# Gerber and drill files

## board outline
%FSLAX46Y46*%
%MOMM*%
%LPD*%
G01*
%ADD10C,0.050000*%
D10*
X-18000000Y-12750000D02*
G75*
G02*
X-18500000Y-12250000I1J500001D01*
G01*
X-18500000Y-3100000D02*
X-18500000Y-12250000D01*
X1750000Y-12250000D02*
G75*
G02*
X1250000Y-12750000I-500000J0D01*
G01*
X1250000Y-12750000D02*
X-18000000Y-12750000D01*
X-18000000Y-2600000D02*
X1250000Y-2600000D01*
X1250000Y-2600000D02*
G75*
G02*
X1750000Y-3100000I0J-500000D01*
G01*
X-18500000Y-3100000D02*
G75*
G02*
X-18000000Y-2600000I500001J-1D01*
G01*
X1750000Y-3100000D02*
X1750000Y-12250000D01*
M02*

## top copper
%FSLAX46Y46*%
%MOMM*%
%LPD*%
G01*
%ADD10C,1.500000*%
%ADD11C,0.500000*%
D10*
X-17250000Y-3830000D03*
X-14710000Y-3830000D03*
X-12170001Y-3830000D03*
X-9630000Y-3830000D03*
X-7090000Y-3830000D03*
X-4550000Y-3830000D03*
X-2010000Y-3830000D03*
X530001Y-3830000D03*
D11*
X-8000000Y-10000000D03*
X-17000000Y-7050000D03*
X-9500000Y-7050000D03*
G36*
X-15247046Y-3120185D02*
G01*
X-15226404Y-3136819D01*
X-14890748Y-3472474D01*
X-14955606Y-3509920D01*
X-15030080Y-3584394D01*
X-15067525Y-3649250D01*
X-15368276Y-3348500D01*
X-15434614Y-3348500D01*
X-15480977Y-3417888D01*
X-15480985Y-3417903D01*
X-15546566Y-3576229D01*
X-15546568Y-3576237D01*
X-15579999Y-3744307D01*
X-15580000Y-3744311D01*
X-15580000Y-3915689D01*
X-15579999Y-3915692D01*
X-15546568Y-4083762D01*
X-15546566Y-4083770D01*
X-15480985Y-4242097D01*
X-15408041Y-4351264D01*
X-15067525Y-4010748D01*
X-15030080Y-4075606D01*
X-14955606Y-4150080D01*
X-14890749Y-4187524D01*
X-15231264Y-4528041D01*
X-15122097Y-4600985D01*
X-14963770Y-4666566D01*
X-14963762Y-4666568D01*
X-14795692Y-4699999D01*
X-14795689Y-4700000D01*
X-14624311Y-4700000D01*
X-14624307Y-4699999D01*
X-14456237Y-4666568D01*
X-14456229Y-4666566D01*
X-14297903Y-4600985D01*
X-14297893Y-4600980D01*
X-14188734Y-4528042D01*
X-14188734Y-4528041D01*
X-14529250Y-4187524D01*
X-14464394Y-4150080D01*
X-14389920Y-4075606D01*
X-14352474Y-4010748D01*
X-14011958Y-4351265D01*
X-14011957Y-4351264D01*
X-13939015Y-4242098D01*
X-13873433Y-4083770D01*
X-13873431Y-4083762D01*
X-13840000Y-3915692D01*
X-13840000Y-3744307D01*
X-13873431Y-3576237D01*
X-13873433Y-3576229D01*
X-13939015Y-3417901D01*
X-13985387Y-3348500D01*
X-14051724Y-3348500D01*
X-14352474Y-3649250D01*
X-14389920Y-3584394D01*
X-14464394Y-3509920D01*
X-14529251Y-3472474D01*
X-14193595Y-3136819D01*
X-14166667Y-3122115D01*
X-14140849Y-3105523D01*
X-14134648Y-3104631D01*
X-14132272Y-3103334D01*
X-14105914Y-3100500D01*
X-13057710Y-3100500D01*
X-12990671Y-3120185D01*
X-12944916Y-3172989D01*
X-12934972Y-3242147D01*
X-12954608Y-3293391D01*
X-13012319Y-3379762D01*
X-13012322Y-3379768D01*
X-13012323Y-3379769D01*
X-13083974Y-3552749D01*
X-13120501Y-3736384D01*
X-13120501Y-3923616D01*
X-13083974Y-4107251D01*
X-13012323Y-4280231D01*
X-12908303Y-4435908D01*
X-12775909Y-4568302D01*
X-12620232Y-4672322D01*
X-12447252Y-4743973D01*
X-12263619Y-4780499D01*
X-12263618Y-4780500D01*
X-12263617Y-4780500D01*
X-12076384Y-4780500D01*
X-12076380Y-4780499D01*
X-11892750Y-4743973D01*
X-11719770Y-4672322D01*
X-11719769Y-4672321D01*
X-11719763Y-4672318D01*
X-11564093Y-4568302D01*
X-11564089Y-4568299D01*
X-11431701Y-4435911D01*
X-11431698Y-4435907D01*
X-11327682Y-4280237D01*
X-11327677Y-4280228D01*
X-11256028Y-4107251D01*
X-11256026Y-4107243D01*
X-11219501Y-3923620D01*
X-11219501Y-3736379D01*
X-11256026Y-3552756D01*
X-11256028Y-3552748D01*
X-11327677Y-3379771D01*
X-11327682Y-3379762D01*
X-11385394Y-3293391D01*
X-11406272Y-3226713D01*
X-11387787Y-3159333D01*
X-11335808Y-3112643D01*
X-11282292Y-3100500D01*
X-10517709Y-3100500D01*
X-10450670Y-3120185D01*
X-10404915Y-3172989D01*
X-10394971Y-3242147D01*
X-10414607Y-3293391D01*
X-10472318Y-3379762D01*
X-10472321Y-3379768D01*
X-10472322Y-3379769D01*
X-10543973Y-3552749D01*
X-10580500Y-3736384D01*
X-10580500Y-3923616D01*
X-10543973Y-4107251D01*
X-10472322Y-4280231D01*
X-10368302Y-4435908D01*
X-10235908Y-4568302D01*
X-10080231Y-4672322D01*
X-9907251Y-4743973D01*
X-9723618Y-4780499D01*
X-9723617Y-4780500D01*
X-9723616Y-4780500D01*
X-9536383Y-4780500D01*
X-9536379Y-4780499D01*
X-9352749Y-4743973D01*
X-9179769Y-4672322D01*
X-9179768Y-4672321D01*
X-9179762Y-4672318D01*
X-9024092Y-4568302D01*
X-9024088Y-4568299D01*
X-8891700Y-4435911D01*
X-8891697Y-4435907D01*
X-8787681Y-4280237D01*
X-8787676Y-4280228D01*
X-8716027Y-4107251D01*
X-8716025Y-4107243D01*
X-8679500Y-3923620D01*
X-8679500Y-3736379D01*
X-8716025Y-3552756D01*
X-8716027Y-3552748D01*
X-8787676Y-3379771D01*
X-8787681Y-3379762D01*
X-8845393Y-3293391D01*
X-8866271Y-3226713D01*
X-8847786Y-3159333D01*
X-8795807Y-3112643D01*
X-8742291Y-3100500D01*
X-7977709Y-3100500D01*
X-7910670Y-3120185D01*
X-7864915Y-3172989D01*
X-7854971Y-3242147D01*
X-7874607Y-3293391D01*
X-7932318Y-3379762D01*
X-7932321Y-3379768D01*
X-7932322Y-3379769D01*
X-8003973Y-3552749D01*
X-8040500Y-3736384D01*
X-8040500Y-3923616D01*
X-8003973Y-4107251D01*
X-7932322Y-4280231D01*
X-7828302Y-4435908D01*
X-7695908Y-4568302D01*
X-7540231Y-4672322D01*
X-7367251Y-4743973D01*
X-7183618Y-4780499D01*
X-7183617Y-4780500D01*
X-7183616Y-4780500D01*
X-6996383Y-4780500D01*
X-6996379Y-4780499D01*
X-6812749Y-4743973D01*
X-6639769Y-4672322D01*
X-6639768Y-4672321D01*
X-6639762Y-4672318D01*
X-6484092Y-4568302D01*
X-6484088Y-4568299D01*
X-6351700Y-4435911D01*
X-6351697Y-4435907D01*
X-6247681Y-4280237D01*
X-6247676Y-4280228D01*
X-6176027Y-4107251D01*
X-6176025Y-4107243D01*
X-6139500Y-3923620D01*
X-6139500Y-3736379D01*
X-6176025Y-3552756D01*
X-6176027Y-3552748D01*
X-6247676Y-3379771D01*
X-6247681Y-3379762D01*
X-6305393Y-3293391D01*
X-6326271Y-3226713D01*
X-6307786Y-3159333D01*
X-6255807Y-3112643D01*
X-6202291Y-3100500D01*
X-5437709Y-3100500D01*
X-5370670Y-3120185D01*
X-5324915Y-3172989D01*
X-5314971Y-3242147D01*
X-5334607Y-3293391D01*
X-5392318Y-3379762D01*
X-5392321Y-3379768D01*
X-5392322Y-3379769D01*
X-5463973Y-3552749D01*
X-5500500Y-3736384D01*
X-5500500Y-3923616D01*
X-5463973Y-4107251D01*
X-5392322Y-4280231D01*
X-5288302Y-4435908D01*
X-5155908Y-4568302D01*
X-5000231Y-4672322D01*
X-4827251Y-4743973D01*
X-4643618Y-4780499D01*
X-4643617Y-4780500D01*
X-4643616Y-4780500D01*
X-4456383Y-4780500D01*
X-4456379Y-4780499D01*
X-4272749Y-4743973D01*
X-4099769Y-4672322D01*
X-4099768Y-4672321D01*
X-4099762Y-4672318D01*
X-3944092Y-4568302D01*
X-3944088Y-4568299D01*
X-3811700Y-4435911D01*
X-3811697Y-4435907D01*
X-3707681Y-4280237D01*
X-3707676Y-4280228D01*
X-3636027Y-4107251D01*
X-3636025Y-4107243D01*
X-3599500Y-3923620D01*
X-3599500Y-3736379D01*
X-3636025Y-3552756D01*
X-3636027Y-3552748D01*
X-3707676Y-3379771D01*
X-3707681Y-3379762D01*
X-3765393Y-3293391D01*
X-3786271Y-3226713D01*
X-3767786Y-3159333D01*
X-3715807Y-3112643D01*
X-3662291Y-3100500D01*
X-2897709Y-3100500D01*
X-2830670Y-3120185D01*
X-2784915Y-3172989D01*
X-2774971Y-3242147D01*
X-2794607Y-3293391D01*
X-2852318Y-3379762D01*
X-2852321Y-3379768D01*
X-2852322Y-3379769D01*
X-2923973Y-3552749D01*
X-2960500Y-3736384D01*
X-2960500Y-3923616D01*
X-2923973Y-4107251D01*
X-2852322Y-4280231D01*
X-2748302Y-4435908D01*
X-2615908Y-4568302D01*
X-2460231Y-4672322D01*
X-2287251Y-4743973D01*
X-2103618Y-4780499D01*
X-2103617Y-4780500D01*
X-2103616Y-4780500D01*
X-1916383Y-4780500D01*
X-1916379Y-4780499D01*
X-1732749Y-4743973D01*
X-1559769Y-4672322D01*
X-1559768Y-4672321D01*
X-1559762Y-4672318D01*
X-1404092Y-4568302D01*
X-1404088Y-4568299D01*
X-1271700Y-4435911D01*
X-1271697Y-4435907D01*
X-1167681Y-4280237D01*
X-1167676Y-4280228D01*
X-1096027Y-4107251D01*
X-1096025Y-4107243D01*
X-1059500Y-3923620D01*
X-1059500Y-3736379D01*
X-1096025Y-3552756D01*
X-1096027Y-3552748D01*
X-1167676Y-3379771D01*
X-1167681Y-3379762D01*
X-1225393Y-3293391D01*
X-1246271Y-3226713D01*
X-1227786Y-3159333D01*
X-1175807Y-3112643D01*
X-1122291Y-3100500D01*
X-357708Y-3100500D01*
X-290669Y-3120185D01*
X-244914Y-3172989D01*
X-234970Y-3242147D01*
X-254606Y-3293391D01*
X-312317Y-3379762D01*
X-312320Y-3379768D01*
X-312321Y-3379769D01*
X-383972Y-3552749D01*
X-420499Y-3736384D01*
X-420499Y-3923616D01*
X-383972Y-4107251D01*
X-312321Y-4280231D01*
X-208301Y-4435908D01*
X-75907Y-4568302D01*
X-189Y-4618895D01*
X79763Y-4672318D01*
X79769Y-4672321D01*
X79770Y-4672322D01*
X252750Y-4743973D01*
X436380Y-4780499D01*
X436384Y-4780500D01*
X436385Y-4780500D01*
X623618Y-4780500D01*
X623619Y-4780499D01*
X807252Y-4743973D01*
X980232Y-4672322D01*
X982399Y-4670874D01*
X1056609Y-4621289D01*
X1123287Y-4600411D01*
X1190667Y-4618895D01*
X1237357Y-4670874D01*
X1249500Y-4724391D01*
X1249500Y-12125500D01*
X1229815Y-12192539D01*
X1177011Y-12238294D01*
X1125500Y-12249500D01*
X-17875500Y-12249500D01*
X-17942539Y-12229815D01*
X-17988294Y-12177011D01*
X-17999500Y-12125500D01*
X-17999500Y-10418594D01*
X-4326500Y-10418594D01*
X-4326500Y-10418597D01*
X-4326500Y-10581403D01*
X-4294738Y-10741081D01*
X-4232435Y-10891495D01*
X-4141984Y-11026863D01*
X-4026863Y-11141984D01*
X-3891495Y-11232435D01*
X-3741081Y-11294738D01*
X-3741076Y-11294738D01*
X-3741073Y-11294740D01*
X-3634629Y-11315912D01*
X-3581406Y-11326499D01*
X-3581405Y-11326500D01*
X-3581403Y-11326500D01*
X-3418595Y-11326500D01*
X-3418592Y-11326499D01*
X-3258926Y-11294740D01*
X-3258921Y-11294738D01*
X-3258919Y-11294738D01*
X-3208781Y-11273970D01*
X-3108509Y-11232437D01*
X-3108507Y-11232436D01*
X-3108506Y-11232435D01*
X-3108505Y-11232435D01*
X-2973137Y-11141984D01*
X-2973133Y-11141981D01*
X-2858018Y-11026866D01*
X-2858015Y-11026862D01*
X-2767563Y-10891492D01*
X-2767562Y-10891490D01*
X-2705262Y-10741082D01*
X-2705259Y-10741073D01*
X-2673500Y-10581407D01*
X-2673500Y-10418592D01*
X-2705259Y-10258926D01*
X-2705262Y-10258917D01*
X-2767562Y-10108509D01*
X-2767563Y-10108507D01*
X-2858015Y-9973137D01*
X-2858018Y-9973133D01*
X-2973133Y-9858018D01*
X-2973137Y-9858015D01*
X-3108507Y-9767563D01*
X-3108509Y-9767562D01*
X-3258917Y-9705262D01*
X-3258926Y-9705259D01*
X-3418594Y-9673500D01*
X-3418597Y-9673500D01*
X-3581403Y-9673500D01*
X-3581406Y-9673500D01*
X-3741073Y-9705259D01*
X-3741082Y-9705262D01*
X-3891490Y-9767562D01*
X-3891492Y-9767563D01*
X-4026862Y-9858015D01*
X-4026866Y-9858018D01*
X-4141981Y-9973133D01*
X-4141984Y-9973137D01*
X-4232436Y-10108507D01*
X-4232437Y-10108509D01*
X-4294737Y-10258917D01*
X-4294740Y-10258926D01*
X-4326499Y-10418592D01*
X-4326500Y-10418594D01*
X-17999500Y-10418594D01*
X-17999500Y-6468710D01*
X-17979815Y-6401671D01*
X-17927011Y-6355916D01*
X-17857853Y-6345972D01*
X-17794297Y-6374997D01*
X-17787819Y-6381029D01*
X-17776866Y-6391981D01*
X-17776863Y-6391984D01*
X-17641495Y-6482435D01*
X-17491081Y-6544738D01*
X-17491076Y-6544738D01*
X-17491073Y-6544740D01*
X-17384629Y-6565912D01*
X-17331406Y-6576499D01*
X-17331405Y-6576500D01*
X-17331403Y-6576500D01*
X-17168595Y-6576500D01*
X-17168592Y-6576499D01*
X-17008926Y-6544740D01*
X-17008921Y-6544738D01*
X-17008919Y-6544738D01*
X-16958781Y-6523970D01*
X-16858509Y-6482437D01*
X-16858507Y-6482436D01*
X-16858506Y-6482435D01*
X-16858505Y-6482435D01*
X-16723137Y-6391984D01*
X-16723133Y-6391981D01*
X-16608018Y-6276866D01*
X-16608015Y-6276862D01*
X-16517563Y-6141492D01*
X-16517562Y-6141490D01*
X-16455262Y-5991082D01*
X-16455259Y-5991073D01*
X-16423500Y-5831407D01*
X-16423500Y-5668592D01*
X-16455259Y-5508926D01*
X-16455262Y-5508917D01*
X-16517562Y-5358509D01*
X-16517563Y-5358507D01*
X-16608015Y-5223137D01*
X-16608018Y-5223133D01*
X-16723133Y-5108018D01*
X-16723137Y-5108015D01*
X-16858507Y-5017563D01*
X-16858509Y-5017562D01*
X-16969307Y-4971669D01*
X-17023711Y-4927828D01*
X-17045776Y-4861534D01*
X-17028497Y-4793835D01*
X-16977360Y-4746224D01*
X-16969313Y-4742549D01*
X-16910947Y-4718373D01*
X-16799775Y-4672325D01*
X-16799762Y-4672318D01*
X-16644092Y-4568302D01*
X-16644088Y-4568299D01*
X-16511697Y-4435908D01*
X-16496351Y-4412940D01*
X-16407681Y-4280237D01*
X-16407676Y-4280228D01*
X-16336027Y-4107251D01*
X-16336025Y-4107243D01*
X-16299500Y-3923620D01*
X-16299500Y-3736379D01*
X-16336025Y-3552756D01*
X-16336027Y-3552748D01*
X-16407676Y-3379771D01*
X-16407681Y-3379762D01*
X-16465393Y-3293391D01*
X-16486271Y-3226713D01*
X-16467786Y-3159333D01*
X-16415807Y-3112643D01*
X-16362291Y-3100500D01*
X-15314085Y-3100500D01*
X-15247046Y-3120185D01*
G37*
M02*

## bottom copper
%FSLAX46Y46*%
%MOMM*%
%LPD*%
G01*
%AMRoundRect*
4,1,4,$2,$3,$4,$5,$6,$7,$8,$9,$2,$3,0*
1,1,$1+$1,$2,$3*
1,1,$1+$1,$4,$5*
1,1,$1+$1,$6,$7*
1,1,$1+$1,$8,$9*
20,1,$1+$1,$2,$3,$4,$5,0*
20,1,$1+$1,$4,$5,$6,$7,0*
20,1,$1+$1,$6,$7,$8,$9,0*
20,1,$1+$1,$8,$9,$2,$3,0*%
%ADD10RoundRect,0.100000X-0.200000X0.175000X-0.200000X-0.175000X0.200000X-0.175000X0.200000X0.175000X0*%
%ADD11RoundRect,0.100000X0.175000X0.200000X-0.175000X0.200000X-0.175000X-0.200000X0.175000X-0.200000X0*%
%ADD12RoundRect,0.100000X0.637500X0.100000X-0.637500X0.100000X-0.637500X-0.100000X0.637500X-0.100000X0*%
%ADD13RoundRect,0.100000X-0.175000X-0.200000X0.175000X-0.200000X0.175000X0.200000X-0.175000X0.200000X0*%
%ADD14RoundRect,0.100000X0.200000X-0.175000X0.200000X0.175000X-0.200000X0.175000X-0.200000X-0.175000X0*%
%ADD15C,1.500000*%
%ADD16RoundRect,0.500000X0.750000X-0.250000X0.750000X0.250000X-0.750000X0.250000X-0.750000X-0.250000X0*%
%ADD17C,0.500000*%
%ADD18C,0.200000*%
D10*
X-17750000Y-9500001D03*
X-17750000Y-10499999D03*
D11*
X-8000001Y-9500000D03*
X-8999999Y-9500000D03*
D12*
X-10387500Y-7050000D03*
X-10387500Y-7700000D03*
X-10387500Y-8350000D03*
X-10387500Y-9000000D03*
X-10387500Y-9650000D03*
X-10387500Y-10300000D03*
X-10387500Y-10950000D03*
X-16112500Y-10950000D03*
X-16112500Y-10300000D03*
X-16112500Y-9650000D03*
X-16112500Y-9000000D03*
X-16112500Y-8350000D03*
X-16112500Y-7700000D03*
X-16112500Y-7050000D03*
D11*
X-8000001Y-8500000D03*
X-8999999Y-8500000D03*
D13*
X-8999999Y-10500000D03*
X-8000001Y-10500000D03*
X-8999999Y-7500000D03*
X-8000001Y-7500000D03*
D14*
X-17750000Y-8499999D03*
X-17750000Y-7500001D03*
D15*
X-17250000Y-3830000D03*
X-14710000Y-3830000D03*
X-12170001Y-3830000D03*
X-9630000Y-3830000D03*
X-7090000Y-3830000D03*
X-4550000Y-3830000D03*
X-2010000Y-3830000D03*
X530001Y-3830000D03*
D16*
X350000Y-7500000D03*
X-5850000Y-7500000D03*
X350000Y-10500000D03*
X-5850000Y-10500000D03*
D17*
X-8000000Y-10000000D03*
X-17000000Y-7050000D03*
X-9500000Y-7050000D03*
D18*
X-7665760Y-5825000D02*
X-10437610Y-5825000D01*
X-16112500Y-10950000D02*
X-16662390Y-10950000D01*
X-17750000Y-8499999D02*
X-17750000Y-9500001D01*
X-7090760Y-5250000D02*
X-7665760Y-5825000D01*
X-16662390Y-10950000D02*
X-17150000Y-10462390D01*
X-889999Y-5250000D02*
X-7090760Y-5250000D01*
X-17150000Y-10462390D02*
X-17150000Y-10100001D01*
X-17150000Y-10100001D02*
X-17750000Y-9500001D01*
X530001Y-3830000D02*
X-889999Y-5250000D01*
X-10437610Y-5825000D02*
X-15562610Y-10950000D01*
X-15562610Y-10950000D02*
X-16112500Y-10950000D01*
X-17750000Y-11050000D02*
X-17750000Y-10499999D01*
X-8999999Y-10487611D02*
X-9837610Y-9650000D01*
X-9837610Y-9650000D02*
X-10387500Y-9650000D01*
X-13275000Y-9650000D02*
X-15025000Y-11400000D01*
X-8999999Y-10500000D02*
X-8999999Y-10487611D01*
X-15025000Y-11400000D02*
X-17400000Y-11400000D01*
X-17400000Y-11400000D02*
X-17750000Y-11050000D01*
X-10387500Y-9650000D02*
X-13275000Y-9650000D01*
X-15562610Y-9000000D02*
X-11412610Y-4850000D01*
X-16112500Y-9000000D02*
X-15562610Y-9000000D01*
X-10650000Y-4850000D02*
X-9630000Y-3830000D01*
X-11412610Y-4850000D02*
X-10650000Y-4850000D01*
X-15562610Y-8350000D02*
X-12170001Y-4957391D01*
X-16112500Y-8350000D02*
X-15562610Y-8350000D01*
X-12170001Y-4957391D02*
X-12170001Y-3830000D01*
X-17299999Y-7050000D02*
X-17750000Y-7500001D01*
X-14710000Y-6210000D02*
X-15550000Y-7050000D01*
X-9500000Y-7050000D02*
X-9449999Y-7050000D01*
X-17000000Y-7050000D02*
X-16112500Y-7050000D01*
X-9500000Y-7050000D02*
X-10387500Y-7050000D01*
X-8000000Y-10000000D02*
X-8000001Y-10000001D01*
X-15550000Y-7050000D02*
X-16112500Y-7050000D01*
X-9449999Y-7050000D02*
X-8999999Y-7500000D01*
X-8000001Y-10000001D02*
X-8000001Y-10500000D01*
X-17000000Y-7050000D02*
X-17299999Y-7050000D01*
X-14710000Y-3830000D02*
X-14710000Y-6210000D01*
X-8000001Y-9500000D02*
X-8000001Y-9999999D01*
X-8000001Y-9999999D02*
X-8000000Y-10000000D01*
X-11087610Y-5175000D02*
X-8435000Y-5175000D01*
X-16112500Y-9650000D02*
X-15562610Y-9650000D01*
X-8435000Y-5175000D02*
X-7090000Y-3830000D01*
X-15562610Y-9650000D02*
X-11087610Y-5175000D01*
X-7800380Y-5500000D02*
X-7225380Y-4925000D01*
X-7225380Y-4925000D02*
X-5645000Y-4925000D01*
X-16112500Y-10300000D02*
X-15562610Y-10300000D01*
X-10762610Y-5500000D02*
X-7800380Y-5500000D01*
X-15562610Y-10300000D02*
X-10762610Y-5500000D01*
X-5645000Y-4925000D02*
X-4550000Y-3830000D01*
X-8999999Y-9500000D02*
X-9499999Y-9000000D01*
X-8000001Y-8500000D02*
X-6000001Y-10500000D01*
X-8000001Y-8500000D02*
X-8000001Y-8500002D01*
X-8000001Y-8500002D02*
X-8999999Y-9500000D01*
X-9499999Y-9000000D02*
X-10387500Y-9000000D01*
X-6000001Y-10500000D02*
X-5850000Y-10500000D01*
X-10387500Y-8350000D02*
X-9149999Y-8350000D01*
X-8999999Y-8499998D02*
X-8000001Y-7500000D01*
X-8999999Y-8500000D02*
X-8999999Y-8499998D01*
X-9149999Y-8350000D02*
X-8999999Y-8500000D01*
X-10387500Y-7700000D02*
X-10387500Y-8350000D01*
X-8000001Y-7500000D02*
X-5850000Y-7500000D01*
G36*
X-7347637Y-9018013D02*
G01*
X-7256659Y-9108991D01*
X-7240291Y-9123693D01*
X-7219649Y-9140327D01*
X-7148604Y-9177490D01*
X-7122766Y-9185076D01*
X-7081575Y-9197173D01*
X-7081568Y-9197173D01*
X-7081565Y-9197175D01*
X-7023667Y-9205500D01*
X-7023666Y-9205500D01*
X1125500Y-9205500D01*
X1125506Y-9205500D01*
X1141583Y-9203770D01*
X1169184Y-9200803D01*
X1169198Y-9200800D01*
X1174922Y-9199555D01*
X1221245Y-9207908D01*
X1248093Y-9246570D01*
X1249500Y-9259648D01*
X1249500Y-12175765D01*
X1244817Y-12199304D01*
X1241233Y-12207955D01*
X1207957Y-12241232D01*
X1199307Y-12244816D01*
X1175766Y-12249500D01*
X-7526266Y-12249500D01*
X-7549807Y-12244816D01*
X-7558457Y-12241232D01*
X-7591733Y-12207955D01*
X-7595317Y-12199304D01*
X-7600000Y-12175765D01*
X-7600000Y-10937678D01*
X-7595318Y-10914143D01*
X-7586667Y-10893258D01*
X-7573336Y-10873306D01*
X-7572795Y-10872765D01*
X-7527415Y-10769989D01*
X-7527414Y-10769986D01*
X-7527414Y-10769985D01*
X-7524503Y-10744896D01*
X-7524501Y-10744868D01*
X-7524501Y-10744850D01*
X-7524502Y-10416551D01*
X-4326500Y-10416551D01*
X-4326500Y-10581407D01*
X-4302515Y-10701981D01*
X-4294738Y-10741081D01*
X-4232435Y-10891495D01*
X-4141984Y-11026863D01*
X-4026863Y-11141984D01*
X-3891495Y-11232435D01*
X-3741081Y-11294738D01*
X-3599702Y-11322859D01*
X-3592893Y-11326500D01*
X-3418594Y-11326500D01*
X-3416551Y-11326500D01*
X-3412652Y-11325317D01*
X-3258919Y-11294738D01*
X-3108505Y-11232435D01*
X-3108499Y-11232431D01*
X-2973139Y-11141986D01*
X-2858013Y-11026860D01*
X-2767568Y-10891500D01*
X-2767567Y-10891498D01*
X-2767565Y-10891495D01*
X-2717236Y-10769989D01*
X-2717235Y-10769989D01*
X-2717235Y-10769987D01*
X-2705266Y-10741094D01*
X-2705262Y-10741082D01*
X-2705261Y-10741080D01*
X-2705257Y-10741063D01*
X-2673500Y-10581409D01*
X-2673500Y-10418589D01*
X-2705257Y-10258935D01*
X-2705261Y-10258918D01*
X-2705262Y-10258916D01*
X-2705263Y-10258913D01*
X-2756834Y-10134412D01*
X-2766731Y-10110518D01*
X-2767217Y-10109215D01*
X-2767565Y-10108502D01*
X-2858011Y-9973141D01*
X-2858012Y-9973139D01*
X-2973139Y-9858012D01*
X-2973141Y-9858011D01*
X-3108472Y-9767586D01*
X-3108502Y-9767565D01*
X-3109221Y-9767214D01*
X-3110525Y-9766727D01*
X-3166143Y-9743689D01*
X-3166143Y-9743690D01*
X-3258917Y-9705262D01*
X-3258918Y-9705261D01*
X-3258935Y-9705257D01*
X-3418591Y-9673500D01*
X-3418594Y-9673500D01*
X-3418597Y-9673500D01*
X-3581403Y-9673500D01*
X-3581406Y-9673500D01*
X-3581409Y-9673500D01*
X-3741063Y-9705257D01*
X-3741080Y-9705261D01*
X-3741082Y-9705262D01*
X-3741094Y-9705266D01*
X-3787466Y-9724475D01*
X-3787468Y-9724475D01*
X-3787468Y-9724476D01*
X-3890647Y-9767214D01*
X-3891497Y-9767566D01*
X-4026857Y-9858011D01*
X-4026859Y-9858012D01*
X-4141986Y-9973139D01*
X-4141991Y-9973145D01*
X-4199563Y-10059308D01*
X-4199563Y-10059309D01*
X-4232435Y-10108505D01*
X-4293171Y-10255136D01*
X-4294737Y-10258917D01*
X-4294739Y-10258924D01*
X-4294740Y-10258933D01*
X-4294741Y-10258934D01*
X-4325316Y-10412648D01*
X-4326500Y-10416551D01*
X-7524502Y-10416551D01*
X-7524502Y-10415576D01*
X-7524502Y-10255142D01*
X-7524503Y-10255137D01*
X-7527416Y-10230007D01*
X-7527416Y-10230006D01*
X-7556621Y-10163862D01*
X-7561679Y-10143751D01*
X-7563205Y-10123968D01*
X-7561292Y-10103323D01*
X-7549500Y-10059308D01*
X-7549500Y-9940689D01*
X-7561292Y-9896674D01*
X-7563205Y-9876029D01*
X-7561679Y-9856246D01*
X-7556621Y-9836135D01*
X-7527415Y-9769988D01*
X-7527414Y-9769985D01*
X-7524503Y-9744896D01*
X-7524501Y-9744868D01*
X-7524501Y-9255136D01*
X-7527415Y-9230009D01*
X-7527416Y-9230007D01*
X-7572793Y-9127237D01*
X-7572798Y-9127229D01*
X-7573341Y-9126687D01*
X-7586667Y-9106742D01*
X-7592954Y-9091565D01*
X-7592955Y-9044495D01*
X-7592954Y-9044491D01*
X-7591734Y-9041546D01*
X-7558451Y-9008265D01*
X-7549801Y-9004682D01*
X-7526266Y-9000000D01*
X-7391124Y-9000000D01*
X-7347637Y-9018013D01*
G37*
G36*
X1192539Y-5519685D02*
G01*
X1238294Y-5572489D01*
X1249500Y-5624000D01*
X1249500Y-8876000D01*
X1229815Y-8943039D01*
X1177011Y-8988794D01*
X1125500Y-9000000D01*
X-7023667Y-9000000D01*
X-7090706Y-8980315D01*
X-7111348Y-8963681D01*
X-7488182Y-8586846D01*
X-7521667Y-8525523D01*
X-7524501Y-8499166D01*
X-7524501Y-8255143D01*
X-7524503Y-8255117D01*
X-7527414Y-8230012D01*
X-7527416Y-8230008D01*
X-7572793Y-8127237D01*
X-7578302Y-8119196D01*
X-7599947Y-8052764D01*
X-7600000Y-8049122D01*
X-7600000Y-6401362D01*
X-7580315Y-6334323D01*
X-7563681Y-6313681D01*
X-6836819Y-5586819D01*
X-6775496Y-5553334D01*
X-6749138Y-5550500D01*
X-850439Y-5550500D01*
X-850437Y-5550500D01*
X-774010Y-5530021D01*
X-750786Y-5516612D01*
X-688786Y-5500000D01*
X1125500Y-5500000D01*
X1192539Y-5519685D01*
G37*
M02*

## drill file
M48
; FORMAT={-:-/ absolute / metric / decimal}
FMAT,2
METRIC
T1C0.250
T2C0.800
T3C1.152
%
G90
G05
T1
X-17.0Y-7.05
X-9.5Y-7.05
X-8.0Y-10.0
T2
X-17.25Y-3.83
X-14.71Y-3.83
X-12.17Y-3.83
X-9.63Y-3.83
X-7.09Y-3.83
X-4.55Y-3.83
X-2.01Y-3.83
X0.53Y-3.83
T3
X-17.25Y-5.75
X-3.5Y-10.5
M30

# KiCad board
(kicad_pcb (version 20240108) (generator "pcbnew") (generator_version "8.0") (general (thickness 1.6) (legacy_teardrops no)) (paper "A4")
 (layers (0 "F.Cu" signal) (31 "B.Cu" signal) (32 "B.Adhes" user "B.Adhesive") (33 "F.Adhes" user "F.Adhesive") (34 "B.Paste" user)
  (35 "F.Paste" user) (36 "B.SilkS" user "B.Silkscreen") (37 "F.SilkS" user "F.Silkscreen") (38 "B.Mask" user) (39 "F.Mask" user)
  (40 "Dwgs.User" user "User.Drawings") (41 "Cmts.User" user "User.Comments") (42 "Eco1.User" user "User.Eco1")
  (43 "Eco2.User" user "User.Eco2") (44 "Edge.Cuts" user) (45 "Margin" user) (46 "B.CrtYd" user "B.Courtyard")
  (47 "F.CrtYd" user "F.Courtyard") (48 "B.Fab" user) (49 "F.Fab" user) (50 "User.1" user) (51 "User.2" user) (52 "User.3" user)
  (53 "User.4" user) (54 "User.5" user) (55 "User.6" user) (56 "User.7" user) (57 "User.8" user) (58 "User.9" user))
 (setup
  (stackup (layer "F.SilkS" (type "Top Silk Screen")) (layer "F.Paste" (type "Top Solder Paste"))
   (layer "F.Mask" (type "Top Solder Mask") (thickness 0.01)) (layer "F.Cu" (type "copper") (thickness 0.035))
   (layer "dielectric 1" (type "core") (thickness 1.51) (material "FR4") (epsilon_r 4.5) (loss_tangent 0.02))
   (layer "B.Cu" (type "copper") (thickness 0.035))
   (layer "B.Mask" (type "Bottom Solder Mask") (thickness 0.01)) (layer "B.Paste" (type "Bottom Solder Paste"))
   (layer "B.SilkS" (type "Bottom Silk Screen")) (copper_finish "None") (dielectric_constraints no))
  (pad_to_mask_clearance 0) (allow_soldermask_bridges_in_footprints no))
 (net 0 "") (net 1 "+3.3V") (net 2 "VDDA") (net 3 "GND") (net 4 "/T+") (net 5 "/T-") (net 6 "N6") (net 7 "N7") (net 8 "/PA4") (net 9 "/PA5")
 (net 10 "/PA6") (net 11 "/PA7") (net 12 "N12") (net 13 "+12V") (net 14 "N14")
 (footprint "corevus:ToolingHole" (layer "F.Cu") (at -17.25 5.75)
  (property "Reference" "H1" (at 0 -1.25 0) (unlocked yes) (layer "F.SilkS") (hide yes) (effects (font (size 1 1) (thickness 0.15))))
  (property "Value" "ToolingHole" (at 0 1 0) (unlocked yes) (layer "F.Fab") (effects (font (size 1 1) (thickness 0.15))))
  (pad "" np_thru_hole circle (at 0 0) (size 1.3 1.3) (drill 1.152) (layers "*.Mask")))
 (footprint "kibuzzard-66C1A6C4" (layer "F.Cu") (at -0.25 7.5)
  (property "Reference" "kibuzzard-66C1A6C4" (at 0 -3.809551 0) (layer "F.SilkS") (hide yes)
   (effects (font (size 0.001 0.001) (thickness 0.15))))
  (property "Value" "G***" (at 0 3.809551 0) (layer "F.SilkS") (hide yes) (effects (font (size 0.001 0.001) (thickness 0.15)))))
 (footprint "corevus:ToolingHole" (layer "F.Cu") (at -3.5 10.5)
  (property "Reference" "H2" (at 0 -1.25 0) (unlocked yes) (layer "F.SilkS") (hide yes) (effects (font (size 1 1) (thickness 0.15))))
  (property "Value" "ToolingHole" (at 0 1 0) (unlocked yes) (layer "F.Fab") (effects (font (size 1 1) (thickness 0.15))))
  (pad "" np_thru_hole circle (at 0 0) (size 1.3 1.3) (drill 1.152) (layers "*.Mask")))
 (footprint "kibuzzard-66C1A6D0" (layer "F.Cu") (at -0.25 10.5)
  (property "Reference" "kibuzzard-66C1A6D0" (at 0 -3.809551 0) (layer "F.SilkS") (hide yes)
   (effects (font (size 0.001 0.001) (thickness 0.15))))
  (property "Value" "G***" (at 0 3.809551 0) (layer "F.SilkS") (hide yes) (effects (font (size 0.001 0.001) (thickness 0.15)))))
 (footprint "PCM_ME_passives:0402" (layer "B.Cu") (at -17.75 10 -90)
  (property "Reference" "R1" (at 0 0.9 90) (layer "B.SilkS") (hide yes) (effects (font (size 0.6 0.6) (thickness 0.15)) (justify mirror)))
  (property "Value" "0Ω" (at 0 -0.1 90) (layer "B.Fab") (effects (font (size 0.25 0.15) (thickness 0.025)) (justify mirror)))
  (pad "1" smd roundrect (at -0.499999 0 270) (size 0.55 0.6) (layers "B.Cu" "B.Paste" "B.Mask") (roundrect_rratio 0.1818181818)
   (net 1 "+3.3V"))
  (pad "2" smd roundrect (at 0.499999 0 270) (size 0.55 0.6) (layers "B.Cu" "B.Paste" "B.Mask") (roundrect_rratio 0.1818181818)
   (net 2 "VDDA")))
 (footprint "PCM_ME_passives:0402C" (layer "B.Cu") (at -8.5 9.5 180)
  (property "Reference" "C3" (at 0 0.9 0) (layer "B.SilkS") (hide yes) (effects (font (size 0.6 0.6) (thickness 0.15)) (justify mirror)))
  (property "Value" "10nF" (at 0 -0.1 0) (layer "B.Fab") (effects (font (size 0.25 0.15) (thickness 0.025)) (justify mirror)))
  (pad "1" smd roundrect (at -0.499999 0 180) (size 0.55 0.6) (layers "B.Cu" "B.Paste" "B.Mask") (roundrect_rratio 0.1818181818)
   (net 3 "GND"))
  (pad "2" smd roundrect (at 0.499999 0 180) (size 0.55 0.6) (layers "B.Cu" "B.Paste" "B.Mask") (roundrect_rratio 0.1818181818)
   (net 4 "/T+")))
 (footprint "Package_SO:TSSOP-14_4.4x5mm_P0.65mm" (layer "B.Cu") (at -13.25 9 180)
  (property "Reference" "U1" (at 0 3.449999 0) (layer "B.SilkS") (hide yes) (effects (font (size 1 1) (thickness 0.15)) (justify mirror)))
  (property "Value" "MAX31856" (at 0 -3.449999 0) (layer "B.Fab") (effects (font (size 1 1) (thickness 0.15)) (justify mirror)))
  (pad "1" smd roundrect (at -2.8625 1.95 180) (size 1.475 0.4) (layers "B.Cu" "B.Paste" "B.Mask") (roundrect_rratio 0.25) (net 3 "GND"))
  (pad "2" smd roundrect (at -2.8625 1.3 180) (size 1.475 0.4) (layers "B.Cu" "B.Paste" "B.Mask") (roundrect_rratio 0.25) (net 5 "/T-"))
  (pad "3" smd roundrect (at -2.8625 0.65 180) (size 1.475 0.4) (layers "B.Cu" "B.Paste" "B.Mask") (roundrect_rratio 0.25) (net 5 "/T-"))
  (pad "4" smd roundrect (at -2.8625 0 180) (size 1.475 0.4) (layers "B.Cu" "B.Paste" "B.Mask") (roundrect_rratio 0.25) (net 4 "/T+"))
  (pad "5" smd roundrect (at -2.8625 -0.65 180) (size 1.475 0.4) (layers "B.Cu" "B.Paste" "B.Mask") (roundrect_rratio 0.25) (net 2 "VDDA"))
  (pad "6" smd roundrect (at -2.8625 -1.3 180) (size 1.475 0.4) (layers "B.Cu" "B.Paste" "B.Mask") (roundrect_rratio 0.25) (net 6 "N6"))
  (pad "7" smd roundrect (at -2.8625 -1.95 180) (size 1.475 0.4) (layers "B.Cu" "B.Paste" "B.Mask") (roundrect_rratio 0.25) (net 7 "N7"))
  (pad "8" smd roundrect (at 2.8625 -1.95 180) (size 1.475 0.4) (layers "B.Cu" "B.Paste" "B.Mask") (roundrect_rratio 0.25) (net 1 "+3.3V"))
  (pad "9" smd roundrect (at 2.8625 -1.3 180) (size 1.475 0.4) (layers "B.Cu" "B.Paste" "B.Mask") (roundrect_rratio 0.25) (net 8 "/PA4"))
  (pad "10" smd roundrect (at 2.8625 -0.65 180) (size 1.475 0.4) (layers "B.Cu" "B.Paste" "B.Mask") (roundrect_rratio 0.25) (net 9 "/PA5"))
  (pad "11" smd roundrect (at 2.8625 0 180) (size 1.475 0.4) (layers "B.Cu" "B.Paste" "B.Mask") (roundrect_rratio 0.25) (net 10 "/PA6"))
  (pad "12" smd roundrect (at 2.8625 0.65 180) (size 1.475 0.4) (layers "B.Cu" "B.Paste" "B.Mask") (roundrect_rratio 0.25) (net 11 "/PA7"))
  (pad "13" smd roundrect (at 2.8625 1.3 180) (size 1.475 0.4) (layers "B.Cu" "B.Paste" "B.Mask") (roundrect_rratio 0.25) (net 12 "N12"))
  (pad "14" smd roundrect (at 2.8625 1.95 180) (size 1.475 0.4) (layers "B.Cu" "B.Paste" "B.Mask") (roundrect_rratio 0.25) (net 3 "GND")))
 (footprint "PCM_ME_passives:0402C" (layer "B.Cu") (at -8.5 8.5 180)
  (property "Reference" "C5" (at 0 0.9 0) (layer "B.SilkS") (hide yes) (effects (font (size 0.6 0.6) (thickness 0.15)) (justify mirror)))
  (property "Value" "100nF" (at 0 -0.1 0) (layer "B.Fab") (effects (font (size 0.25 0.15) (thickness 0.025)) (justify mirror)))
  (pad "1" smd roundrect (at -0.499999 0 180) (size 0.55 0.6) (layers "B.Cu" "B.Paste" "B.Mask") (roundrect_rratio 0.1818181818)
   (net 4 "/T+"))
  (pad "2" smd roundrect (at 0.499999 0 180) (size 0.55 0.6) (layers "B.Cu" "B.Paste" "B.Mask") (roundrect_rratio 0.1818181818)
   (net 5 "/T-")))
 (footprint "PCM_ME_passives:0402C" (layer "B.Cu") (at -8.5 10.5)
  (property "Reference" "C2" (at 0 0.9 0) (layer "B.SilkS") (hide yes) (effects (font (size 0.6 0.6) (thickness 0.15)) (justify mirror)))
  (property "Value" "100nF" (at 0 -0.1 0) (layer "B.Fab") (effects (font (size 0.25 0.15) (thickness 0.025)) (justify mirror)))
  (pad "1" smd roundrect (at -0.499999 0) (size 0.55 0.6) (layers "B.Cu" "B.Paste" "B.Mask") (roundrect_rratio 0.1818181818) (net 2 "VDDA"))
  (pad "2" smd roundrect (at 0.499999 0) (size 0.55 0.6) (layers "B.Cu" "B.Paste" "B.Mask") (roundrect_rratio 0.1818181818) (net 3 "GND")))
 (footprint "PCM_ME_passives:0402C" (layer "B.Cu") (at -8.5 7.5)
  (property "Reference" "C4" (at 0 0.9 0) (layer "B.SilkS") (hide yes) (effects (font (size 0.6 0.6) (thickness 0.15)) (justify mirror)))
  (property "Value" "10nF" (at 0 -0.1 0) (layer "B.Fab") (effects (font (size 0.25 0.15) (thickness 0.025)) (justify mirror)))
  (pad "1" smd roundrect (at -0.499999 0) (size 0.55 0.6) (layers "B.Cu" "B.Paste" "B.Mask") (roundrect_rratio 0.1818181818) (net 3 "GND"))
  (pad "2" smd roundrect (at 0.499999 0) (size 0.55 0.6) (layers "B.Cu" "B.Paste" "B.Mask") (roundrect_rratio 0.1818181818) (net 5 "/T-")))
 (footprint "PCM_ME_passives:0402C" (layer "B.Cu") (at -17.75 8 90)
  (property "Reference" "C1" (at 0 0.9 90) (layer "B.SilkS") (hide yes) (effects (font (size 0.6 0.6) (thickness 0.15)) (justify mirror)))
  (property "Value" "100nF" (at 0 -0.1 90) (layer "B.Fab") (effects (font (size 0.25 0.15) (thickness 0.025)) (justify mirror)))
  (pad "1" smd roundrect (at -0.499999 0 90) (size 0.55 0.6) (layers "B.Cu" "B.Paste" "B.Mask") (roundrect_rratio 0.1818181818)
   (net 1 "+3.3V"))
  (pad "2" smd roundrect (at 0.499999 0 90) (size 0.55 0.6) (layers "B.Cu" "B.Paste" "B.Mask") (roundrect_rratio 0.1818181818) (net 3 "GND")))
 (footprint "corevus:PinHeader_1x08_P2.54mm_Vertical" (layer "B.Cu") (at -17.25 3.83 -90)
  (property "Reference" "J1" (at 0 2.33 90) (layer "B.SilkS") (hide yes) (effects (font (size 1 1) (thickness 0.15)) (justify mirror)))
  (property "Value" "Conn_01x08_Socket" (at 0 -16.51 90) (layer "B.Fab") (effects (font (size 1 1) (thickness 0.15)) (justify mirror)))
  (pad "1" thru_hole circle (at 0 0 270) (size 1.5 1.5) (drill 0.8) (layers "*.Cu" "*.Mask") (remove_unused_layers yes)
   (keep_end_layers yes) (zone_layer_connections) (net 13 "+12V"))
  (pad "2" thru_hole circle (at 0 -2.54 270) (size 1.5 1.5) (drill 0.8) (layers "*.Cu" "*.Mask") (remove_unused_layers yes)
   (keep_end_layers yes) (zone_layer_connections) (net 3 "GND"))
  (pad "3" thru_hole circle (at 0 -5.079999 270) (size 1.5 1.5) (drill 0.8) (layers "*.Cu" "*.Mask") (remove_unused_layers yes)
   (keep_end_layers yes) (zone_layer_connections) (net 11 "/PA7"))
  (pad "4" thru_hole circle (at 0 -7.62 270) (size 1.5 1.5) (drill 0.8) (layers "*.Cu" "*.Mask") (remove_unused_layers yes)
   (keep_end_layers yes) (zone_layer_connections) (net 10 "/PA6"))
  (pad "5" thru_hole circle (at 0 -10.16 270) (size 1.5 1.5) (drill 0.8) (layers "*.Cu" "*.Mask") (remove_unused_layers yes)
   (keep_end_layers yes) (zone_layer_connections) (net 9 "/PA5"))
  (pad "6" thru_hole circle (at 0 -12.7 270) (size 1.5 1.5) (drill 0.8) (layers "*.Cu" "*.Mask") (remove_unused_layers yes)
   (keep_end_layers yes) (zone_layer_connections) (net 8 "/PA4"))
  (pad "7" thru_hole circle (at 0 -15.24 270) (size 1.5 1.5) (drill 0.8) (layers "*.Cu" "*.Mask") (remove_unused_layers yes)
   (keep_end_layers yes) (zone_layer_connections) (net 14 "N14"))
  (pad "8" thru_hole circle (at 0 -17.780001 270) (size 1.5 1.5) (drill 0.8) (layers "*.Cu" "*.Mask") (remove_unused_layers yes)
   (keep_end_layers yes) (zone_layer_connections) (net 1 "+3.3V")))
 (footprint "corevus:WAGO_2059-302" (layer "B.Cu") (at -2.5 9 180)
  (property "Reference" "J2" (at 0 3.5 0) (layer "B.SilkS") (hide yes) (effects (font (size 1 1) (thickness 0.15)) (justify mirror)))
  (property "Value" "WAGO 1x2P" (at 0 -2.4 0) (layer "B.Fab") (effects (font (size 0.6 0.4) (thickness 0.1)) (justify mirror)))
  (pad "1" smd roundrect (at -2.85 1.5 90) (size 1.5 2.5) (layers "B.Cu" "B.Paste" "B.Mask") (roundrect_rratio 0.3333333333) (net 5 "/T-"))
  (pad "1" smd roundrect (at 3.35 1.5 90) (size 1.5 2.5) (layers "B.Cu" "B.Paste" "B.Mask") (roundrect_rratio 0.3333333333) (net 5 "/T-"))
  (pad "2" smd roundrect (at -2.85 -1.5 90) (size 1.5 2.5) (layers "B.Cu" "B.Paste" "B.Mask") (roundrect_rratio 0.3333333333) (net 4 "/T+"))
  (pad "2" smd roundrect (at 3.35 -1.5 90) (size 1.5 2.5) (layers "B.Cu" "B.Paste" "B.Mask") (roundrect_rratio 0.3333333333) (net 4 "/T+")))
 (gr_arc (start -18 12.75) (mid -18.353553 12.603553) (end -18.5 12.25) (stroke (width 0.05) (type default)) (layer "Edge.Cuts"))
 (gr_line (start -18.5 3.1) (end -18.5 12.25) (stroke (width 0.05) (type default)) (layer "Edge.Cuts"))
 (gr_arc (start 1.75 12.25) (mid 1.603553 12.603553) (end 1.25 12.75) (stroke (width 0.05) (type default)) (layer "Edge.Cuts"))
 (gr_line (start 1.25 12.75) (end -18 12.75) (stroke (width 0.05) (type default)) (layer "Edge.Cuts"))
 (gr_line (start -18 2.6) (end 1.25 2.6) (stroke (width 0.05) (type default)) (layer "Edge.Cuts"))
 (gr_arc (start 1.25 2.6) (mid 1.603553 2.746447) (end 1.75 3.1) (stroke (width 0.05) (type default)) (layer "Edge.Cuts"))
 (gr_arc (start -18.5 3.1) (mid -18.353553 2.746447) (end -18 2.6) (stroke (width 0.05) (type default)) (layer "Edge.Cuts"))
 (gr_line (start 1.75 3.1) (end 1.75 12.25) (stroke (width 0.05) (type default)) (layer "Edge.Cuts"))
 (segment (start -7.66576 5.825) (end -10.43761 5.825) (width 0.2) (layer "B.Cu") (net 1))
 (segment (start -16.1125 10.95) (end -16.66239 10.95) (width 0.2) (layer "B.Cu") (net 1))
 (segment (start -17.75 8.499999) (end -17.75 9.500001) (width 0.2) (layer "B.Cu") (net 1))
 (segment (start -7.09076 5.25) (end -7.66576 5.825) (width 0.2) (layer "B.Cu") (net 1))
 (segment (start -16.66239 10.95) (end -17.15 10.46239) (width 0.2) (layer "B.Cu") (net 1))
 (segment (start -0.889999 5.25) (end -7.09076 5.25) (width 0.2) (layer "B.Cu") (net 1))
 (segment (start -17.15 10.46239) (end -17.15 10.100001) (width 0.2) (layer "B.Cu") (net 1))
 (segment (start -17.15 10.100001) (end -17.75 9.500001) (width 0.2) (layer "B.Cu") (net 1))
 (segment (start 0.530001 3.83) (end -0.889999 5.25) (width 0.2) (layer "B.Cu") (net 1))
 (segment (start -10.43761 5.825) (end -15.56261 10.95) (width 0.2) (layer "B.Cu") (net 1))
 (segment (start -15.56261 10.95) (end -16.1125 10.95) (width 0.2) (layer "B.Cu") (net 1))
 (segment (start -17.75 11.05) (end -17.75 10.499999) (width 0.2) (layer "B.Cu") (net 2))
 (segment (start -8.999999 10.487611) (end -9.83761 9.65) (width 0.2) (layer "B.Cu") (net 2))
 (segment (start -9.83761 9.65) (end -10.3875 9.65) (width 0.2) (layer "B.Cu") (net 2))
 (segment (start -13.275 9.65) (end -15.025 11.4) (width 0.2) (layer "B.Cu") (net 2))
 (segment (start -8.999999 10.5) (end -8.999999 10.487611) (width 0.2) (layer "B.Cu") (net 2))
 (segment (start -15.025 11.4) (end -17.4 11.4) (width 0.2) (layer "B.Cu") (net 2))
 (segment (start -17.4 11.4) (end -17.75 11.05) (width 0.2) (layer "B.Cu") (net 2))
 (segment (start -10.3875 9.65) (end -13.275 9.65) (width 0.2) (layer "B.Cu") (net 2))
 (segment (start -15.56261 9) (end -11.41261 4.85) (width 0.2) (layer "B.Cu") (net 10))
 (segment (start -16.1125 9) (end -15.56261 9) (width 0.2) (layer "B.Cu") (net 10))
 (segment (start -10.65 4.85) (end -9.63 3.83) (width 0.2) (layer "B.Cu") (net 10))
 (segment (start -11.41261 4.85) (end -10.65 4.85) (width 0.2) (layer "B.Cu") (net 10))
 (segment (start -15.56261 8.35) (end -12.170001 4.957391) (width 0.2) (layer "B.Cu") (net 11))
 (segment (start -16.1125 8.35) (end -15.56261 8.35) (width 0.2) (layer "B.Cu") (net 11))
 (segment (start -12.170001 4.957391) (end -12.170001 3.83) (width 0.2) (layer "B.Cu") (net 11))
 (via (at -8 10) (size 0.5) (drill 0.25) (layers "F.Cu" "B.Cu") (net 3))
 (via (at -17 7.05) (size 0.5) (drill 0.25) (layers "F.Cu" "B.Cu") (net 3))
 (via (at -9.5 7.05) (size 0.5) (drill 0.25) (layers "F.Cu" "B.Cu") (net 3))
 (segment (start -17.299999 7.05) (end -17.75 7.500001) (width 0.2) (layer "B.Cu") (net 3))
 (segment (start -14.71 6.21) (end -15.55 7.05) (width 0.2) (layer "B.Cu") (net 3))
 (segment (start -9.5 7.05) (end -9.449999 7.05) (width 0.2) (layer "B.Cu") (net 3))
 (segment (start -17 7.05) (end -16.1125 7.05) (width 0.2) (layer "B.Cu") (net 3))
 (segment (start -9.5 7.05) (end -10.3875 7.05) (width 0.2) (layer "B.Cu") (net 3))
 (segment (start -8 10) (end -8.000001 10.000001) (width 0.2) (layer "B.Cu") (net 3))
 (segment (start -15.55 7.05) (end -16.1125 7.05) (width 0.2) (layer "B.Cu") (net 3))
 (segment (start -9.449999 7.05) (end -8.999999 7.5) (width 0.2) (layer "B.Cu") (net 3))
 (segment (start -8.000001 10.000001) (end -8.000001 10.5) (width 0.2) (layer "B.Cu") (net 3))
 (segment (start -17 7.05) (end -17.299999 7.05) (width 0.2) (layer "B.Cu") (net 3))
 (segment (start -14.71 3.83) (end -14.71 6.21) (width 0.2) (layer "B.Cu") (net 3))
 (segment (start -8.000001 9.5) (end -8.000001 9.999999) (width 0.2) (layer "B.Cu") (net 3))
 (segment (start -8.000001 9.999999) (end -8 10) (width 0.2) (layer "B.Cu") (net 3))
 (segment (start -11.08761 5.175) (end -8.435 5.175) (width 0.2) (layer "B.Cu") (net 9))
 (segment (start -16.1125 9.65) (end -15.56261 9.65) (width 0.2) (layer "B.Cu") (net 9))
 (segment (start -8.435 5.175) (end -7.09 3.83) (width 0.2) (layer "B.Cu") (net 9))
 (segment (start -15.56261 9.65) (end -11.08761 5.175) (width 0.2) (layer "B.Cu") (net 9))
 (segment (start -7.80038 5.5) (end -7.22538 4.925) (width 0.2) (layer "B.Cu") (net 8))
 (segment (start -7.22538 4.925) (end -5.645 4.925) (width 0.2) (layer "B.Cu") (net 8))
 (segment (start -16.1125 10.3) (end -15.56261 10.3) (width 0.2) (layer "B.Cu") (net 8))
 (segment (start -10.76261 5.5) (end -7.80038 5.5) (width 0.2) (layer "B.Cu") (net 8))
 (segment (start -15.56261 10.3) (end -10.76261 5.5) (width 0.2) (layer "B.Cu") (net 8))
 (segment (start -5.645 4.925) (end -4.55 3.83) (width 0.2) (layer "B.Cu") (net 8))
 (segment (start -8.999999 9.5) (end -9.499999 9) (width 0.2) (layer "B.Cu") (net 4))
 (segment (start -8.000001 8.5) (end -6.000001 10.5) (width 0.2) (layer "B.Cu") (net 4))
 (segment (start -8.000001 8.5) (end -8.000001 8.500002) (width 0.2) (layer "B.Cu") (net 4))
 (segment (start -8.000001 8.500002) (end -8.999999 9.5) (width 0.2) (layer "B.Cu") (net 4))
 (segment (start -9.499999 9) (end -10.3875 9) (width 0.2) (layer "B.Cu") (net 4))
 (segment (start -6.000001 10.5) (end -5.85 10.5) (width 0.2) (layer "B.Cu") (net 4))
 (segment (start -10.3875 8.35) (end -9.149999 8.35) (width 0.2) (layer "B.Cu") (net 5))
 (segment (start -8.999999 8.499998) (end -8.000001 7.5) (width 0.2) (layer "B.Cu") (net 5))
 (segment (start -8.999999 8.5) (end -8.999999 8.499998) (width 0.2) (layer "B.Cu") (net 5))
 (segment (start -9.149999 8.35) (end -8.999999 8.5) (width 0.2) (layer "B.Cu") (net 5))
 (segment (start -10.3875 7.7) (end -10.3875 8.35) (width 0.2) (layer "B.Cu") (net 5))
 (segment (start -8.000001 7.5) (end -5.85 7.5) (width 0.2) (layer "B.Cu") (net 5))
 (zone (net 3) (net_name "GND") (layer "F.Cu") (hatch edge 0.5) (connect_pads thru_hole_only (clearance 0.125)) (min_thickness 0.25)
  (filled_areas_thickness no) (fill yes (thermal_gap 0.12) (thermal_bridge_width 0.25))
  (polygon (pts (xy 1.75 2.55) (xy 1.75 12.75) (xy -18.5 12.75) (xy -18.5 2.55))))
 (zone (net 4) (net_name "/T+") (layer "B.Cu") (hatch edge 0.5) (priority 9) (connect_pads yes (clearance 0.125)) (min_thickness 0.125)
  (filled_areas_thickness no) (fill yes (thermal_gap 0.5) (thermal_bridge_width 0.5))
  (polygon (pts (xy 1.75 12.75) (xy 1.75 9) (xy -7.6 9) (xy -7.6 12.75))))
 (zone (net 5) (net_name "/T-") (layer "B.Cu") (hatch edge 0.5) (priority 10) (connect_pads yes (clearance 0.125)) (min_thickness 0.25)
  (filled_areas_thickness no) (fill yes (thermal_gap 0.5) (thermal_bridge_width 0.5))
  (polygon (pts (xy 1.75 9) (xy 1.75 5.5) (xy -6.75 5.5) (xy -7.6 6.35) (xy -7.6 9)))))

